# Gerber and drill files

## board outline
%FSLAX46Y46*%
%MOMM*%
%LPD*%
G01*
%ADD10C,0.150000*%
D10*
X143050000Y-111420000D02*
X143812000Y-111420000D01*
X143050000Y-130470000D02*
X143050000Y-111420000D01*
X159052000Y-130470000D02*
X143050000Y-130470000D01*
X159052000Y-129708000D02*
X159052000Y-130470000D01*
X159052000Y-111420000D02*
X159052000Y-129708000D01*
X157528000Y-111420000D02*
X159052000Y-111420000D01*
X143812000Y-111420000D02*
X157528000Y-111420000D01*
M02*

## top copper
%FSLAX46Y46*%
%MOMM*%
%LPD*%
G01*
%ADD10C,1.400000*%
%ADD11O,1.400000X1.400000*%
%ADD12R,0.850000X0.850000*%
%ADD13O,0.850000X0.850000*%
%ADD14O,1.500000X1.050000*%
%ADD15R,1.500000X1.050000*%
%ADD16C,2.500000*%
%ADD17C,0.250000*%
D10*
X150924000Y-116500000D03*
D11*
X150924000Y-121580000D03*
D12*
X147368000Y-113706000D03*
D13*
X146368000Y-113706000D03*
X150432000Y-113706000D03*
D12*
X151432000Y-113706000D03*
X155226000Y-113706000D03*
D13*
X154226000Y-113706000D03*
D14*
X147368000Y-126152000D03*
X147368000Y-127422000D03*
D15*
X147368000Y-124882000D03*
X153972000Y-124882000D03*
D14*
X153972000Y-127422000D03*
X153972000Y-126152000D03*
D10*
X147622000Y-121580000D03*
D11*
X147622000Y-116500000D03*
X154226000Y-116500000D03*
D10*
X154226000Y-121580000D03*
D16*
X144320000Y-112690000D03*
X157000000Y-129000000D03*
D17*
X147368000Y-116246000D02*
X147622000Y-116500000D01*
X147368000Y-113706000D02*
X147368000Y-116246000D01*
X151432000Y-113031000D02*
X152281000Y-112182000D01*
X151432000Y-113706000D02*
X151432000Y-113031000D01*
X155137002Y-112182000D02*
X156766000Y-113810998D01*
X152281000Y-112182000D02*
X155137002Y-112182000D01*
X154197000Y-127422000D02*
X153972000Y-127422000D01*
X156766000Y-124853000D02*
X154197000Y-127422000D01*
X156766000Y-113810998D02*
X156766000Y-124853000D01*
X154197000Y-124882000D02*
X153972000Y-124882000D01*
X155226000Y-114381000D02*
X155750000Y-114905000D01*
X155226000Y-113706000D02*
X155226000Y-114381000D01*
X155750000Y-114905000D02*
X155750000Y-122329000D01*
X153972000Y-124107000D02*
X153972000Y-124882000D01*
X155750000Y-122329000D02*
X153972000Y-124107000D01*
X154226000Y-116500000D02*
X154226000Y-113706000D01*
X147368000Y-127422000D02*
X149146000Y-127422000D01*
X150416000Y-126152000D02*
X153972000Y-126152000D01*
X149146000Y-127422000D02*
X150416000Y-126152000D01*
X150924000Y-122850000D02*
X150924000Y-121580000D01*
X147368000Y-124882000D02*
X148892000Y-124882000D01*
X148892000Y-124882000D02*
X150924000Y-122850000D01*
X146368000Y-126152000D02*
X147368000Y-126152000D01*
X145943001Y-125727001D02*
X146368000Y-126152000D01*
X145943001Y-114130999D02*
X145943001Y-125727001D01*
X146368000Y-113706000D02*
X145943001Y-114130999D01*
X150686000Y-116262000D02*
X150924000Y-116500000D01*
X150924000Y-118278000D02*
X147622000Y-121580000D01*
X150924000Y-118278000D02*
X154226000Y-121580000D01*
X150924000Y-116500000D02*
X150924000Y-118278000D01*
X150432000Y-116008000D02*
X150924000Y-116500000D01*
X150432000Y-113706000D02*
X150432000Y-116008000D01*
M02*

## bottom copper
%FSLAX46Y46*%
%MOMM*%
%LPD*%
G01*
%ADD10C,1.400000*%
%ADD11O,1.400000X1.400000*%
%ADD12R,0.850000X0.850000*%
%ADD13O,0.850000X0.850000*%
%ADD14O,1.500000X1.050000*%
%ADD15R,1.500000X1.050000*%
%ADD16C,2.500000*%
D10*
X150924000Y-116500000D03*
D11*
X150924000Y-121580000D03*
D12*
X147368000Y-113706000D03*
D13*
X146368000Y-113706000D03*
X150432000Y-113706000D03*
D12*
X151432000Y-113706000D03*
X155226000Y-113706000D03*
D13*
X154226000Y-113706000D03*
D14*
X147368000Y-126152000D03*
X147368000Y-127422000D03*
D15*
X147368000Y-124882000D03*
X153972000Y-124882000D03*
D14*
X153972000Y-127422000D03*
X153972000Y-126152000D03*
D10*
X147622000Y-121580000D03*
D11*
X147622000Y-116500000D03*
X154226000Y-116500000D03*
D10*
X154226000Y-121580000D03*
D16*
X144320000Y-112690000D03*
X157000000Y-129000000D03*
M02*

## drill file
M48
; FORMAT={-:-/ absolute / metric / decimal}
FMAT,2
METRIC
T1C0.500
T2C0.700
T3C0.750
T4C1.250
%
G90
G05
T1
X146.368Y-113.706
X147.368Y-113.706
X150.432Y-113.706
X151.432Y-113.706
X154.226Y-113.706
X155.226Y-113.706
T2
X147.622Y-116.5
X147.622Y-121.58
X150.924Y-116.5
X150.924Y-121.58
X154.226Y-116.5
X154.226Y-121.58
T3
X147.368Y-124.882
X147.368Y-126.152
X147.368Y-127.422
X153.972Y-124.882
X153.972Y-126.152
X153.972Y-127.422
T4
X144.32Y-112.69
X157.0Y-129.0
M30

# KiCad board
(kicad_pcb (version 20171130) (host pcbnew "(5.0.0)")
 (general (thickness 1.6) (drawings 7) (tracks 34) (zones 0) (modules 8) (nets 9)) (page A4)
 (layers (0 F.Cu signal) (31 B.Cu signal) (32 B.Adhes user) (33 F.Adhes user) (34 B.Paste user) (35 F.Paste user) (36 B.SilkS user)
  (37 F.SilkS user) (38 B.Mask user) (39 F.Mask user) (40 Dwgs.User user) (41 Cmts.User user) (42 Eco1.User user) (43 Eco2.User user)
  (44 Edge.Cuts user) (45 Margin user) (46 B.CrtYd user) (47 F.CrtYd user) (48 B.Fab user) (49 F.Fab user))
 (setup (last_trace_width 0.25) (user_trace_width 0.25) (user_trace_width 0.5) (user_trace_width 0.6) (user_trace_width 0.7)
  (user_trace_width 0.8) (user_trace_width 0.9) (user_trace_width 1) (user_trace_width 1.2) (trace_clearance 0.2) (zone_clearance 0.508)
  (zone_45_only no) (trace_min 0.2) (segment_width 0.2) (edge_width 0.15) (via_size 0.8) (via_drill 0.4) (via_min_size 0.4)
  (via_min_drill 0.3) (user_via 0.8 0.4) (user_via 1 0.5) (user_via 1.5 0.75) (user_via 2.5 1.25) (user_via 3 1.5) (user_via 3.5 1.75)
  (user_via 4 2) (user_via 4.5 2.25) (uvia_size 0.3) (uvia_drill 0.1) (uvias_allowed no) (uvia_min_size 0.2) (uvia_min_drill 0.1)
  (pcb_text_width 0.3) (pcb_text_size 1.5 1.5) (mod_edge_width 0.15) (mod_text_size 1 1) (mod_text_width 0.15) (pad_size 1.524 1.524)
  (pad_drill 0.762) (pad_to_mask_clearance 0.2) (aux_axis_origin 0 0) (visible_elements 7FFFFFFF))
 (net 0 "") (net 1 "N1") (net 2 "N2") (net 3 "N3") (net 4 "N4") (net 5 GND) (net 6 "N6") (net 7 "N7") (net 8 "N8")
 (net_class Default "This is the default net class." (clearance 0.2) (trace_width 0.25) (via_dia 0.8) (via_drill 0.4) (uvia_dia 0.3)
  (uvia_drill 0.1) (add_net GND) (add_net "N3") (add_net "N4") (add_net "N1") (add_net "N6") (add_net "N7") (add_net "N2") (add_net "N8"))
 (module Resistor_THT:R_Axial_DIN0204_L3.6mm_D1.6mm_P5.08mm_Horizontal (layer F.Cu) (at 150.924 116.5 270)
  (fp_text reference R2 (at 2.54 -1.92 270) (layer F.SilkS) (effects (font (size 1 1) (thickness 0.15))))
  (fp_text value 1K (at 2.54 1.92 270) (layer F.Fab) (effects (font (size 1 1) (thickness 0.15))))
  (pad 1 thru_hole circle (at 0 0 270) (size 1.4 1.4) (drill 0.7) (layers *.Cu *.Mask) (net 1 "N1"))
  (pad 2 thru_hole oval (at 5.08 0 270) (size 1.4 1.4) (drill 0.7) (layers *.Cu *.Mask) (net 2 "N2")))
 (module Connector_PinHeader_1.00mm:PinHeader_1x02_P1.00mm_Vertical (layer F.Cu) (at 147.368 113.706 270)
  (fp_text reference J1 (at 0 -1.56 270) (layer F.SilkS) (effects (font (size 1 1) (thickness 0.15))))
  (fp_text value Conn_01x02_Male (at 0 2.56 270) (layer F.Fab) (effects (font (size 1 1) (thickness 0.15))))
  (pad 1 thru_hole rect (at 0 0 270) (size 0.85 0.85) (drill 0.5) (layers *.Cu *.Mask) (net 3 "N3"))
  (pad 2 thru_hole oval (at 0 1 270) (size 0.85 0.85) (drill 0.5) (layers *.Cu *.Mask) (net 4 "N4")))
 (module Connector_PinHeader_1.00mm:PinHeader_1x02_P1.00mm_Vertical (layer F.Cu) (at 151.432 113.706 270)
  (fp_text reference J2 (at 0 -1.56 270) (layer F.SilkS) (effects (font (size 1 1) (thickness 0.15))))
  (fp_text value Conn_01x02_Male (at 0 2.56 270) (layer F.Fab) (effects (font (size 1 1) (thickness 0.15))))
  (pad 2 thru_hole oval (at 0 1 270) (size 0.85 0.85) (drill 0.5) (layers *.Cu *.Mask) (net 1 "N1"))
  (pad 1 thru_hole rect (at 0 0 270) (size 0.85 0.85) (drill 0.5) (layers *.Cu *.Mask) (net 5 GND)))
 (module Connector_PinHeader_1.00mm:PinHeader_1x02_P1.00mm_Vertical (layer F.Cu) (at 155.226 113.706 270)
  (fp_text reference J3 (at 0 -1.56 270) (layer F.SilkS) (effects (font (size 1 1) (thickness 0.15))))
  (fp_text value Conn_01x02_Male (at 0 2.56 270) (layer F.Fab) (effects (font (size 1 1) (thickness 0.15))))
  (pad 1 thru_hole rect (at 0 0 270) (size 0.85 0.85) (drill 0.5) (layers *.Cu *.Mask) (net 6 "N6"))
  (pad 2 thru_hole oval (at 0 1 270) (size 0.85 0.85) (drill 0.5) (layers *.Cu *.Mask) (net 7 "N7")))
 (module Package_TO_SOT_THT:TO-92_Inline (layer F.Cu) (at 147.368 124.882 270)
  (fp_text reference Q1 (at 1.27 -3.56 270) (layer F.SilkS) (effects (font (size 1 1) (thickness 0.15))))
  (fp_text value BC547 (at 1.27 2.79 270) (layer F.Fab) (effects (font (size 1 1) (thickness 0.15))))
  (pad 2 thru_hole oval (at 1.27 0 270) (size 1.05 1.5) (drill 0.75) (layers *.Cu *.Mask) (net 4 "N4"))
  (pad 3 thru_hole oval (at 2.54 0 270) (size 1.05 1.5) (drill 0.75) (layers *.Cu *.Mask) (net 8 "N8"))
  (pad 1 thru_hole rect (at 0 0 270) (size 1.05 1.5) (drill 0.75) (layers *.Cu *.Mask) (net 2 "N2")))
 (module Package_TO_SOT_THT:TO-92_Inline (layer F.Cu) (at 153.972 124.882 270)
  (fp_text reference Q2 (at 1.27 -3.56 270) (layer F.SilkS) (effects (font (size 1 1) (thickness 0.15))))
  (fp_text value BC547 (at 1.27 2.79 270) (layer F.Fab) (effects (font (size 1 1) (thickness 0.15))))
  (pad 1 thru_hole rect (at 0 0 270) (size 1.05 1.5) (drill 0.75) (layers *.Cu *.Mask) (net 6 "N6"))
  (pad 3 thru_hole oval (at 2.54 0 270) (size 1.05 1.5) (drill 0.75) (layers *.Cu *.Mask) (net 5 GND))
  (pad 2 thru_hole oval (at 1.27 0 270) (size 1.05 1.5) (drill 0.75) (layers *.Cu *.Mask) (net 8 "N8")))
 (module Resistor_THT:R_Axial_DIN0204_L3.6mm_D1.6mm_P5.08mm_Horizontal (layer F.Cu) (at 147.622 121.58 90)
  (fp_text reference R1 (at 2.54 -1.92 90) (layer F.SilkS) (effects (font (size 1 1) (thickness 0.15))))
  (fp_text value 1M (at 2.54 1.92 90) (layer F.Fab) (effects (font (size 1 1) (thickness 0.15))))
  (pad 1 thru_hole circle (at 0 0 90) (size 1.4 1.4) (drill 0.7) (layers *.Cu *.Mask) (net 1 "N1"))
  (pad 2 thru_hole oval (at 5.08 0 90) (size 1.4 1.4) (drill 0.7) (layers *.Cu *.Mask) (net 3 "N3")))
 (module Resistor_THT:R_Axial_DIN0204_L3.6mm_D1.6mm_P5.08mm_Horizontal (layer F.Cu) (at 154.226 121.58 90)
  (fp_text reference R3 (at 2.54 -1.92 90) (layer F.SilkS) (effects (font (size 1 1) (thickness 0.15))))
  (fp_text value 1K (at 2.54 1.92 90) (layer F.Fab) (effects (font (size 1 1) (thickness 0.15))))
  (pad 2 thru_hole oval (at 5.08 0 90) (size 1.4 1.4) (drill 0.7) (layers *.Cu *.Mask) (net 7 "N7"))
  (pad 1 thru_hole circle (at 0 0 90) (size 1.4 1.4) (drill 0.7) (layers *.Cu *.Mask) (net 1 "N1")))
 (gr_line (start 143.05 111.42) (end 143.812 111.42) (layer Edge.Cuts) (width 0.15))
 (gr_line (start 143.05 130.47) (end 143.05 111.42) (layer Edge.Cuts) (width 0.15))
 (gr_line (start 159.052 130.47) (end 143.05 130.47) (layer Edge.Cuts) (width 0.15))
 (gr_line (start 159.052 129.708) (end 159.052 130.47) (layer Edge.Cuts) (width 0.15))
 (gr_line (start 159.052 111.42) (end 159.052 129.708) (layer Edge.Cuts) (width 0.15))
 (gr_line (start 157.528 111.42) (end 159.052 111.42) (layer Edge.Cuts) (width 0.15))
 (gr_line (start 143.812 111.42) (end 157.528 111.42) (layer Edge.Cuts) (width 0.15))
 (via (at 144.32 112.69) (size 2.5) (drill 1.25) (layers F.Cu B.Cu) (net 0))
 (via (at 157 129) (size 2.5) (drill 1.25) (layers F.Cu B.Cu) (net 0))
 (segment (start 147.368 116.246) (end 147.622 116.5) (width 0.25) (layer F.Cu) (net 3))
 (segment (start 147.368 113.706) (end 147.368 116.246) (width 0.25) (layer F.Cu) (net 3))
 (segment (start 151.432 113.031) (end 152.281 112.182) (width 0.25) (layer F.Cu) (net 5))
 (segment (start 151.432 113.706) (end 151.432 113.031) (width 0.25) (layer F.Cu) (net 5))
 (segment (start 155.137002 112.182) (end 156.766 113.810998) (width 0.25) (layer F.Cu) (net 5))
 (segment (start 152.281 112.182) (end 155.137002 112.182) (width 0.25) (layer F.Cu) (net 5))
 (segment (start 154.197 127.422) (end 153.972 127.422) (width 0.25) (layer F.Cu) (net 5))
 (segment (start 156.766 124.853) (end 154.197 127.422) (width 0.25) (layer F.Cu) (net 5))
 (segment (start 156.766 113.810998) (end 156.766 124.853) (width 0.25) (layer F.Cu) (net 5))
 (segment (start 154.197 124.882) (end 153.972 124.882) (width 0.25) (layer F.Cu) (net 6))
 (segment (start 155.226 114.381) (end 155.75 114.905) (width 0.25) (layer F.Cu) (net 6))
 (segment (start 155.226 113.706) (end 155.226 114.381) (width 0.25) (layer F.Cu) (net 6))
 (segment (start 155.75 114.905) (end 155.75 122.329) (width 0.25) (layer F.Cu) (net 6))
 (segment (start 153.972 124.107) (end 153.972 124.882) (width 0.25) (layer F.Cu) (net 6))
 (segment (start 155.75 122.329) (end 153.972 124.107) (width 0.25) (layer F.Cu) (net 6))
 (segment (start 154.226 116.5) (end 154.226 113.706) (width 0.25) (layer F.Cu) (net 7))
 (segment (start 147.368 127.422) (end 149.146 127.422) (width 0.25) (layer F.Cu) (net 8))
 (segment (start 150.416 126.152) (end 153.972 126.152) (width 0.25) (layer F.Cu) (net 8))
 (segment (start 149.146 127.422) (end 150.416 126.152) (width 0.25) (layer F.Cu) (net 8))
 (segment (start 150.924 122.85) (end 150.924 121.58) (width 0.25) (layer F.Cu) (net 2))
 (segment (start 147.368 124.882) (end 148.892 124.882) (width 0.25) (layer F.Cu) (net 2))
 (segment (start 148.892 124.882) (end 150.924 122.85) (width 0.25) (layer F.Cu) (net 2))
 (segment (start 146.368 126.152) (end 147.368 126.152) (width 0.25) (layer F.Cu) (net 4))
 (segment (start 145.943001 125.727001) (end 146.368 126.152) (width 0.25) (layer F.Cu) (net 4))
 (segment (start 145.943001 114.130999) (end 145.943001 125.727001) (width 0.25) (layer F.Cu) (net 4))
 (segment (start 146.368 113.706) (end 145.943001 114.130999) (width 0.25) (layer F.Cu) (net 4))
 (segment (start 150.686 116.262) (end 150.924 116.5) (width 0.25) (layer F.Cu) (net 1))
 (segment (start 150.924 118.278) (end 147.622 121.58) (width 0.25) (layer F.Cu) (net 1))
 (segment (start 150.924 118.278) (end 154.226 121.58) (width 0.25) (layer F.Cu) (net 1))
 (segment (start 150.924 116.5) (end 150.924 118.278) (width 0.25) (layer F.Cu) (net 1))
 (segment (start 150.432 116.008) (end 150.924 116.5) (width 0.25) (layer F.Cu) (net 1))
 (segment (start 150.432 113.706) (end 150.432 116.008) (width 0.25) (layer F.Cu) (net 1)))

